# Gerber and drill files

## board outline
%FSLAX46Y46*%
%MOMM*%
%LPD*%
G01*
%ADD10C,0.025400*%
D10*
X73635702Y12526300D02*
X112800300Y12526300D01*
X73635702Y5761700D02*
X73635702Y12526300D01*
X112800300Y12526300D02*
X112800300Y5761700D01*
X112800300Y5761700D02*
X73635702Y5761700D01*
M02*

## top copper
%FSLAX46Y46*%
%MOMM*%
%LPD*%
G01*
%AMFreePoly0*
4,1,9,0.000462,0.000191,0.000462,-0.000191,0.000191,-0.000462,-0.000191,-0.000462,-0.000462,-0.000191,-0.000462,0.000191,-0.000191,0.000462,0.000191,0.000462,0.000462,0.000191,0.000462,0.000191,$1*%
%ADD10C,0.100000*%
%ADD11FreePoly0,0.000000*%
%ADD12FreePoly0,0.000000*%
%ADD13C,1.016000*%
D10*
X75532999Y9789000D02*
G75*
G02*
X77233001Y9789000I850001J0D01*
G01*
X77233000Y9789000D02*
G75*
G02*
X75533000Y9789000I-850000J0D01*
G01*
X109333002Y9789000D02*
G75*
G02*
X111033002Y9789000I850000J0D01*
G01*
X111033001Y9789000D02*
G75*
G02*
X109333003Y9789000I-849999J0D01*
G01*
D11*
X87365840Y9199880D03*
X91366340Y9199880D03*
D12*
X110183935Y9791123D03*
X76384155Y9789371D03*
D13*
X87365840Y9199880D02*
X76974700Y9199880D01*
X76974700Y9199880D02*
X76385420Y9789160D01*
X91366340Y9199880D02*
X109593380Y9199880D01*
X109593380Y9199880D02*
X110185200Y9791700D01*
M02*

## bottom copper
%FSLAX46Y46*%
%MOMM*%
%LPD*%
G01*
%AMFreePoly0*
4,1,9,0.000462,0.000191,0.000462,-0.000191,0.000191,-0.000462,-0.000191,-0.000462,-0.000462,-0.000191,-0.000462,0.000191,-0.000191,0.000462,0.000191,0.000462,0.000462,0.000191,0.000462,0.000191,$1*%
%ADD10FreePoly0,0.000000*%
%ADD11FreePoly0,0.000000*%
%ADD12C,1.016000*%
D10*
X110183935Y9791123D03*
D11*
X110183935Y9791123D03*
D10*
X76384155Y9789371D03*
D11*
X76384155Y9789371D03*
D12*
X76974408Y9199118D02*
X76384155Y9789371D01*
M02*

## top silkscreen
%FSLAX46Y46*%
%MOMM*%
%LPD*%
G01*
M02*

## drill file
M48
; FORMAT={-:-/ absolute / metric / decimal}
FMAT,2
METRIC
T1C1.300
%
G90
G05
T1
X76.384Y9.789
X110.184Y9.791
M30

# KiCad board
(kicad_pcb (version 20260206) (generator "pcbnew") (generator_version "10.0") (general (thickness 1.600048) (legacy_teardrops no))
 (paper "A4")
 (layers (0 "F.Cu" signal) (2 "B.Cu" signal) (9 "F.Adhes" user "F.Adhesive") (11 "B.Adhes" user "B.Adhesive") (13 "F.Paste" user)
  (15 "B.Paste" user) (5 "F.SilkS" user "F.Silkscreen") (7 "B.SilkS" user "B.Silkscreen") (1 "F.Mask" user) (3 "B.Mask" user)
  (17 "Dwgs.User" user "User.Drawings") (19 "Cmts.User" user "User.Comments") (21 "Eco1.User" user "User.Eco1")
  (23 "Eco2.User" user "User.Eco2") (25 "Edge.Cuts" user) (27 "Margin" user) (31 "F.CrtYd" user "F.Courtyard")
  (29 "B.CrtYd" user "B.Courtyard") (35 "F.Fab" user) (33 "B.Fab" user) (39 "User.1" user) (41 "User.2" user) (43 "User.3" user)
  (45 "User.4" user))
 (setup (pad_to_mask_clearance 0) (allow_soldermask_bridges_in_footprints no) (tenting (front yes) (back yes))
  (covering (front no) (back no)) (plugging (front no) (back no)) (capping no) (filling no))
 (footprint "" (layer "F.Cu") (at 0 0)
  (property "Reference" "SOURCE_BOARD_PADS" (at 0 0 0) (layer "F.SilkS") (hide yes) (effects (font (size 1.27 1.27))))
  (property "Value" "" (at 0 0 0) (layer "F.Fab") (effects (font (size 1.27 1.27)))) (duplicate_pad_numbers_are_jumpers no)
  (pad "1" smd custom (at 87.36584 -9.19988) (size 0.001 0.001) (layers "F.Cu" "F.Mask" "F.Paste") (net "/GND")
   (options (clearance outline) (anchor circle)) (primitives))
  (pad "2" smd custom (at 91.36634 -9.19988) (size 0.001 0.001) (layers "F.Cu" "F.Mask" "F.Paste") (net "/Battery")
   (options (clearance outline) (anchor circle)) (primitives)))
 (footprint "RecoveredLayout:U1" (layer "B.Cu") (at 110.183935 -9.791123)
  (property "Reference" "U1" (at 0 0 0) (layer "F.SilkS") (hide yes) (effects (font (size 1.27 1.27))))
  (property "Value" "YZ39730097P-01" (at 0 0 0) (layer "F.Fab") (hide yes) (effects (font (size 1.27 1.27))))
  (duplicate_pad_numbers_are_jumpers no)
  (pad "1" thru_hole custom (at 0 0) (size 0.001 0.001) (drill 1.300023) (layers "*.Cu") (remove_unused_layers no) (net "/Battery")
   (options (clearance outline) (anchor circle)) (primitives))
  (pad "1" smd custom (at 0 0) (size 0.001 0.001) (layers "B.Cu" "B.Mask" "B.Paste") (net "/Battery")
   (options (clearance outline) (anchor circle)) (primitives)))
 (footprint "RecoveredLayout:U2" (layer "B.Cu") (at 76.384155 -9.789371)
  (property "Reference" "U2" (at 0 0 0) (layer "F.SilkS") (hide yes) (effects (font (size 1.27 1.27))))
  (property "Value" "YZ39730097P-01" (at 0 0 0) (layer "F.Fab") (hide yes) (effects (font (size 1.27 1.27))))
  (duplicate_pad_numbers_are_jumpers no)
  (pad "1" thru_hole custom (at 0 0) (size 0.001 0.001) (drill 1.300023) (layers "*.Cu") (remove_unused_layers no) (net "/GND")
   (options (clearance outline) (anchor circle)) (primitives))
  (pad "1" smd custom (at 0 0) (size 0.001 0.001) (layers "B.Cu" "B.Mask" "B.Paste") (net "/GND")
   (options (clearance outline) (anchor circle)) (primitives)))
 (gr_arc (start 75.532999 -9.789) (mid 76.401288 -10.638804) (end 77.233 -9.789) (stroke (width 0.1) (type default)) (layer "F.Cu")
  (net "/GND"))
 (gr_arc (start 77.233 -9.789) (mid 76.364711 -8.939196) (end 75.532999 -9.789) (stroke (width 0.1) (type default)) (layer "F.Cu")
  (net "/GND"))
 (gr_arc (start 109.333002 -9.789) (mid 110.20129 -10.638803) (end 111.033001 -9.789) (stroke (width 0.1) (type default)) (layer "F.Cu")
  (net "/Battery"))
 (gr_arc (start 111.033001 -9.789) (mid 110.164713 -8.939197) (end 109.333002 -9.789) (stroke (width 0.1) (type default)) (layer "F.Cu")
  (net "/Battery"))
 (gr_line (start 73.635702 -12.5263) (end 112.8003 -12.5263) (stroke (width 0.0254) (type default)) (layer "Edge.Cuts"))
 (gr_line (start 73.635702 -5.7617) (end 73.635702 -12.5263) (stroke (width 0.0254) (type default)) (layer "Edge.Cuts"))
 (gr_line (start 112.8003 -12.5263) (end 112.8003 -5.7617) (stroke (width 0.0254) (type default)) (layer "Edge.Cuts"))
 (gr_line (start 112.8003 -5.7617) (end 73.635702 -5.7617) (stroke (width 0.0254) (type default)) (layer "Edge.Cuts"))
 (segment (start 87.36584 -9.19988) (end 76.9747 -9.19988) (width 1.016) (layer "F.Cu") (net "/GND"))
 (segment (start 76.9747 -9.19988) (end 76.38542 -9.78916) (width 1.016) (layer "F.Cu") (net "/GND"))
 (segment (start 76.974408 -9.199118) (end 76.384155 -9.789371) (width 1.016) (layer "B.Cu") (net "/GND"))
 (segment (start 91.36634 -9.19988) (end 109.59338 -9.19988) (width 1.016) (layer "F.Cu") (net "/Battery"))
 (segment (start 109.59338 -9.19988) (end 110.1852 -9.7917) (width 1.016) (layer "F.Cu") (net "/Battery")))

